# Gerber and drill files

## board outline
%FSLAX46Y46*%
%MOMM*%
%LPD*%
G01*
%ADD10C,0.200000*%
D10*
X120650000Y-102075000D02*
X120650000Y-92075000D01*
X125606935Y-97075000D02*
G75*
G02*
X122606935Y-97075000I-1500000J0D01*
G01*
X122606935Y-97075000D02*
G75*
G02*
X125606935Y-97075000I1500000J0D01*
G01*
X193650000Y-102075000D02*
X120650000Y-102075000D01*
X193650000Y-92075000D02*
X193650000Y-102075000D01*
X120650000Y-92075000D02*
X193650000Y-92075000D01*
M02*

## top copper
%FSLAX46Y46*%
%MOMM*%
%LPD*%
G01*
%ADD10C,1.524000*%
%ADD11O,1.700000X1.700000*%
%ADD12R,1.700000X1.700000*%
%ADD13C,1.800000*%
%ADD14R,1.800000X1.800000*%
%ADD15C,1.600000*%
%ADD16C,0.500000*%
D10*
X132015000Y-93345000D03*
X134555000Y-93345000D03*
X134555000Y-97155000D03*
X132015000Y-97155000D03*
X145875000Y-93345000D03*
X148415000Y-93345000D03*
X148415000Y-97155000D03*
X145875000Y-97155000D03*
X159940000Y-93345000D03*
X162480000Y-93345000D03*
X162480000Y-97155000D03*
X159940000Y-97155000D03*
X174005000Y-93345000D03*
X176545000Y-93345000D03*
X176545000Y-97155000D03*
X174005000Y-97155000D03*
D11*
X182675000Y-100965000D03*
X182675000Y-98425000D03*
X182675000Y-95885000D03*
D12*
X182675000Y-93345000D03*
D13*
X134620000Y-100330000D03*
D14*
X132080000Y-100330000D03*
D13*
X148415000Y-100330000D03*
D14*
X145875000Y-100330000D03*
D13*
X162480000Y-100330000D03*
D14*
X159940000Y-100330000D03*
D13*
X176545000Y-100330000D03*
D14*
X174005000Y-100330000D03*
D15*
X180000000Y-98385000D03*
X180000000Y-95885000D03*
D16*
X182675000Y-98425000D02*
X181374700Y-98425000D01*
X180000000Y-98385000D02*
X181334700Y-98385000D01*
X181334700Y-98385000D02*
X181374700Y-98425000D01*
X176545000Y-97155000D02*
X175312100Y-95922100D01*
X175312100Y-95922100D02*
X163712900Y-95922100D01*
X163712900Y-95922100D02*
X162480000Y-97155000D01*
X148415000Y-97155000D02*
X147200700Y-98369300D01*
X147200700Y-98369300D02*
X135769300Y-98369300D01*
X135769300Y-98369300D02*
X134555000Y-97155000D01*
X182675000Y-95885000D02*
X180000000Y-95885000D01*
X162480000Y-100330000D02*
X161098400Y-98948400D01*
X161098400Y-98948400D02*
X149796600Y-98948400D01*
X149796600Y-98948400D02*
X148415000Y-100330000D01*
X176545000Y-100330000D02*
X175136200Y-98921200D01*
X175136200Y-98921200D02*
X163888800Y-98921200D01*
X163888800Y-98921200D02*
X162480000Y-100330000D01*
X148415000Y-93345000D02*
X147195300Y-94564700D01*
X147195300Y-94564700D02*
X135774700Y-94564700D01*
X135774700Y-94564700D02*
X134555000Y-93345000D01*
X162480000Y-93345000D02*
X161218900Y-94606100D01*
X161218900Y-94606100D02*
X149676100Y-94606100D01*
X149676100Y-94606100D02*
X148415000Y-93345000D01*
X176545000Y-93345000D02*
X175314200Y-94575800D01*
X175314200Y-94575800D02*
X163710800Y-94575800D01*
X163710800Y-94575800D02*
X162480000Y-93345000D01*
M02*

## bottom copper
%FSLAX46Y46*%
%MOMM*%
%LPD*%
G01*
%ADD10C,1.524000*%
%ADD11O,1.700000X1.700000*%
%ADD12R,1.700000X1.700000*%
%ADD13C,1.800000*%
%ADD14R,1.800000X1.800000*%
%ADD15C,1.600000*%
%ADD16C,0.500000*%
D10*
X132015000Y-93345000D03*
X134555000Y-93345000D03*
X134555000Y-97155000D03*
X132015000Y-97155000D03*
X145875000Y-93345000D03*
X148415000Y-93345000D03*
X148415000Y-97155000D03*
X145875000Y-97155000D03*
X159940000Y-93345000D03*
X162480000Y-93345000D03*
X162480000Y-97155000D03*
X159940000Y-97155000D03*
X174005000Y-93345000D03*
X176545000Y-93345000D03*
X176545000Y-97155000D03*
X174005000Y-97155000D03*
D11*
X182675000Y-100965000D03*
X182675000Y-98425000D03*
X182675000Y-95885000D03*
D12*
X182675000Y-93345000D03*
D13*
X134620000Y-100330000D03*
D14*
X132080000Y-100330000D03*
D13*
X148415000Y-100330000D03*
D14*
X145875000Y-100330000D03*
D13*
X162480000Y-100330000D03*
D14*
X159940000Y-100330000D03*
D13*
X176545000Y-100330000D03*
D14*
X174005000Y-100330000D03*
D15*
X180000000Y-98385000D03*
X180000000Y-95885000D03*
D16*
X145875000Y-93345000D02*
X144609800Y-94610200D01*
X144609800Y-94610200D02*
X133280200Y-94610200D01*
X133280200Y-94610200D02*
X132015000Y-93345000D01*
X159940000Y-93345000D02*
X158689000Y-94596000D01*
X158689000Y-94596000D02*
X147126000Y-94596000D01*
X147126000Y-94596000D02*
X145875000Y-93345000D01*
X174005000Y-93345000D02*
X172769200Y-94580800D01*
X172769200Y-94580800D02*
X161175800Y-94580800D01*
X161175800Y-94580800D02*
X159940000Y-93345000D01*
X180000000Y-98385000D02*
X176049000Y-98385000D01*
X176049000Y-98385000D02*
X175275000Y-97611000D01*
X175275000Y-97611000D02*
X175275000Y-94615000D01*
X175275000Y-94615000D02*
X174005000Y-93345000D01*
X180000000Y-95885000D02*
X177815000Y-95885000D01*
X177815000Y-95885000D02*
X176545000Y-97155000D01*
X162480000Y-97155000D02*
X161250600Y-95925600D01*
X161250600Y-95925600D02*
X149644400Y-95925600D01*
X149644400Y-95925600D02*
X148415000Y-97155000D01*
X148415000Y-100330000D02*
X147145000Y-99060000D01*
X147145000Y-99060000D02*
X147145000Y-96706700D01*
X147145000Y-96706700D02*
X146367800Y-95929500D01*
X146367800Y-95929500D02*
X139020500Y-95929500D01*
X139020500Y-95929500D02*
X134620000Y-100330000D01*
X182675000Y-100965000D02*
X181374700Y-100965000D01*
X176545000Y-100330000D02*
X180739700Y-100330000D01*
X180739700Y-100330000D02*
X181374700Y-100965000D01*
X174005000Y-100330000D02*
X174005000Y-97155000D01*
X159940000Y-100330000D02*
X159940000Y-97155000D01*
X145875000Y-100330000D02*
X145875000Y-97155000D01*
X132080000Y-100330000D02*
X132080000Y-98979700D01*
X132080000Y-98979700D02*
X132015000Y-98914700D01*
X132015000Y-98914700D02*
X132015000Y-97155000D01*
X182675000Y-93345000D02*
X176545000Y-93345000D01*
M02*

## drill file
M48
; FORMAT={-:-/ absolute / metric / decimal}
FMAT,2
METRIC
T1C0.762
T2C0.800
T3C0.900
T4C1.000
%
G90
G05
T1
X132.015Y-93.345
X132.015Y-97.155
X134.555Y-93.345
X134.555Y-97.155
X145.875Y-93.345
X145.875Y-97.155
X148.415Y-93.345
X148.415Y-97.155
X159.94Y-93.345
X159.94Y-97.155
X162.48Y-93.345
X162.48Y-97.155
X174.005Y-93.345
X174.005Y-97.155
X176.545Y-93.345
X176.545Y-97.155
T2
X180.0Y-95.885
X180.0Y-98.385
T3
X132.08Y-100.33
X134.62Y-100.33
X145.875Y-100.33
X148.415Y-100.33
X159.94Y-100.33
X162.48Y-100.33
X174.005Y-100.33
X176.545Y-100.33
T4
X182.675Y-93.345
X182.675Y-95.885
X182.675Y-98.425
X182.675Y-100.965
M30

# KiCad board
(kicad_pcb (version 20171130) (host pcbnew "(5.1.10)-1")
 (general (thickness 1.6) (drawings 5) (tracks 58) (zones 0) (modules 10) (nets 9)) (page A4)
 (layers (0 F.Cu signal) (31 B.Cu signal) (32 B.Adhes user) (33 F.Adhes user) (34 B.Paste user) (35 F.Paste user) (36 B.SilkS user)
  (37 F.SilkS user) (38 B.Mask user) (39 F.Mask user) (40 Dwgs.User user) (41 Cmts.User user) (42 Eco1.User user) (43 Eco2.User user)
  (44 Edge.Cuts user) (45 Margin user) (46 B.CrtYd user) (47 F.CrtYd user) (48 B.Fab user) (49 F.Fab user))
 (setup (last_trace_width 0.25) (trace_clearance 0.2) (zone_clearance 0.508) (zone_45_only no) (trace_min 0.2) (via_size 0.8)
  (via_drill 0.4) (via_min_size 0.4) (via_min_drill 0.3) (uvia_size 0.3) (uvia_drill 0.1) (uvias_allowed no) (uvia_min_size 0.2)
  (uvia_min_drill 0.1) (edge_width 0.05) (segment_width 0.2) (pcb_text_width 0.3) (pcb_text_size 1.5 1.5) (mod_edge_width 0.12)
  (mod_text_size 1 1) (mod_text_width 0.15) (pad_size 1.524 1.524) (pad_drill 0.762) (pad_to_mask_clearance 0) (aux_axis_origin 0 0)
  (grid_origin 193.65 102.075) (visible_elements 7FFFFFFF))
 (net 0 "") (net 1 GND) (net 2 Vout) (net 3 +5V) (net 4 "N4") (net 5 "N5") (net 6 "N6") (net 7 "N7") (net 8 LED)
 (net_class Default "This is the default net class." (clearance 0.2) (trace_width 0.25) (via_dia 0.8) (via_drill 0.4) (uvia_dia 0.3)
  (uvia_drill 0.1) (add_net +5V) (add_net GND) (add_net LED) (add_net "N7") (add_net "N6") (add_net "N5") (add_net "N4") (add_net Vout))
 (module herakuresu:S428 (layer F.Cu) (at 133.285 94.615 180)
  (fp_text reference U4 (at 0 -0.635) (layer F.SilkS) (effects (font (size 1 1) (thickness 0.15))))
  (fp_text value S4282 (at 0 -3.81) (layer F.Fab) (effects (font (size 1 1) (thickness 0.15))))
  (pad 4 thru_hole circle (at 1.27 1.27 180) (size 1.524 1.524) (drill 0.762) (layers *.Cu *.Mask) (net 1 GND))
  (pad 3 thru_hole circle (at -1.27 1.27 180) (size 1.524 1.524) (drill 0.762) (layers *.Cu *.Mask) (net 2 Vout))
  (pad 2 thru_hole circle (at -1.27 -2.54 180) (size 1.524 1.524) (drill 0.762) (layers *.Cu *.Mask) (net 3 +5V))
  (pad 1 thru_hole circle (at 1.27 -2.54 180) (size 1.524 1.524) (drill 0.762) (layers *.Cu *.Mask) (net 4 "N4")))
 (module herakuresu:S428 (layer F.Cu) (at 147.145 94.615 180)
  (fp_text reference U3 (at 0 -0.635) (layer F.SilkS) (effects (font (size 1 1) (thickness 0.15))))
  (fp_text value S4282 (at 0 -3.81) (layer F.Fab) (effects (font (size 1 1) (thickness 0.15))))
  (pad 4 thru_hole circle (at 1.27 1.27 180) (size 1.524 1.524) (drill 0.762) (layers *.Cu *.Mask) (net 1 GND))
  (pad 3 thru_hole circle (at -1.27 1.27 180) (size 1.524 1.524) (drill 0.762) (layers *.Cu *.Mask) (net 2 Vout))
  (pad 2 thru_hole circle (at -1.27 -2.54 180) (size 1.524 1.524) (drill 0.762) (layers *.Cu *.Mask) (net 3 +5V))
  (pad 1 thru_hole circle (at 1.27 -2.54 180) (size 1.524 1.524) (drill 0.762) (layers *.Cu *.Mask) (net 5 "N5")))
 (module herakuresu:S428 (layer F.Cu) (at 161.21 94.615 180)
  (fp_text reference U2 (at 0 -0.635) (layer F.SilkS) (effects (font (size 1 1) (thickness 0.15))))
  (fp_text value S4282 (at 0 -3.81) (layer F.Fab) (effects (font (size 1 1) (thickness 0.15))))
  (pad 4 thru_hole circle (at 1.27 1.27 180) (size 1.524 1.524) (drill 0.762) (layers *.Cu *.Mask) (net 1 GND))
  (pad 3 thru_hole circle (at -1.27 1.27 180) (size 1.524 1.524) (drill 0.762) (layers *.Cu *.Mask) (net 2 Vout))
  (pad 2 thru_hole circle (at -1.27 -2.54 180) (size 1.524 1.524) (drill 0.762) (layers *.Cu *.Mask) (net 3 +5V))
  (pad 1 thru_hole circle (at 1.27 -2.54 180) (size 1.524 1.524) (drill 0.762) (layers *.Cu *.Mask) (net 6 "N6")))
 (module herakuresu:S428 (layer F.Cu) (at 175.275 94.615 180)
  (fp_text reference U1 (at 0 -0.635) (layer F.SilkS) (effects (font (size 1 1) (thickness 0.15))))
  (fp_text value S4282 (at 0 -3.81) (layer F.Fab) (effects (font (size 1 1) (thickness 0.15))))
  (pad 4 thru_hole circle (at 1.27 1.27 180) (size 1.524 1.524) (drill 0.762) (layers *.Cu *.Mask) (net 1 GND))
  (pad 3 thru_hole circle (at -1.27 1.27 180) (size 1.524 1.524) (drill 0.762) (layers *.Cu *.Mask) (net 2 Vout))
  (pad 2 thru_hole circle (at -1.27 -2.54 180) (size 1.524 1.524) (drill 0.762) (layers *.Cu *.Mask) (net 3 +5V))
  (pad 1 thru_hole circle (at 1.27 -2.54 180) (size 1.524 1.524) (drill 0.762) (layers *.Cu *.Mask) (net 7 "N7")))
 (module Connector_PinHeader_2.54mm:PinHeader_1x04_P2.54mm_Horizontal (layer F.Cu) (at 182.675 93.345)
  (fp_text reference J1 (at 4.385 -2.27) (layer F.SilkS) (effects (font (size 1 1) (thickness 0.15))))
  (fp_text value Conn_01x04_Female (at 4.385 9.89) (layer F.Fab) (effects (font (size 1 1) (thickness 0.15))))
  (pad 4 thru_hole oval (at 0 7.62) (size 1.7 1.7) (drill 1) (layers *.Cu *.Mask) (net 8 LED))
  (pad 3 thru_hole oval (at 0 5.08) (size 1.7 1.7) (drill 1) (layers *.Cu *.Mask) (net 1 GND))
  (pad 2 thru_hole oval (at 0 2.54) (size 1.7 1.7) (drill 1) (layers *.Cu *.Mask) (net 3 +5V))
  (pad 1 thru_hole rect (at 0 0) (size 1.7 1.7) (drill 1) (layers *.Cu *.Mask) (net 2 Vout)))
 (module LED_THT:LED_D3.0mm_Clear (layer F.Cu) (at 132.08 100.33)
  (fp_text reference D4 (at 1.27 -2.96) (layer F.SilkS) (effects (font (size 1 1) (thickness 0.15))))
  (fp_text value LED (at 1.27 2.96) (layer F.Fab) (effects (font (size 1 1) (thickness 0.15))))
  (pad 2 thru_hole circle (at 2.54 0) (size 1.8 1.8) (drill 0.9) (layers *.Cu *.Mask) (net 8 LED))
  (pad 1 thru_hole rect (at 0 0) (size 1.8 1.8) (drill 0.9) (layers *.Cu *.Mask) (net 4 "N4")))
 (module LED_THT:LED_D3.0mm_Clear (layer F.Cu) (at 145.875 100.33)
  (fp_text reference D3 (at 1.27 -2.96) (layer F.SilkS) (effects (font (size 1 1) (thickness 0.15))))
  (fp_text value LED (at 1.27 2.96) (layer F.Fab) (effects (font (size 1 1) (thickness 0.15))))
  (pad 2 thru_hole circle (at 2.54 0) (size 1.8 1.8) (drill 0.9) (layers *.Cu *.Mask) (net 8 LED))
  (pad 1 thru_hole rect (at 0 0) (size 1.8 1.8) (drill 0.9) (layers *.Cu *.Mask) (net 5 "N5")))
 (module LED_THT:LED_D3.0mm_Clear (layer F.Cu) (at 159.94 100.33)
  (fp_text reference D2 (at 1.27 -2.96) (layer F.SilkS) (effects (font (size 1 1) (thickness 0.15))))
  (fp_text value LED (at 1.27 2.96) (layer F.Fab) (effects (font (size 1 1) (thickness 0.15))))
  (pad 2 thru_hole circle (at 2.54 0) (size 1.8 1.8) (drill 0.9) (layers *.Cu *.Mask) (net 8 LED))
  (pad 1 thru_hole rect (at 0 0) (size 1.8 1.8) (drill 0.9) (layers *.Cu *.Mask) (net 6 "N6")))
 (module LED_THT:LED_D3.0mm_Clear (layer F.Cu) (at 174.005 100.33)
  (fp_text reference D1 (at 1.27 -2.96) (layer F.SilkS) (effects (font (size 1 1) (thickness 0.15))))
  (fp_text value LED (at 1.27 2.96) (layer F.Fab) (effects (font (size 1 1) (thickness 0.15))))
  (pad 2 thru_hole circle (at 2.54 0) (size 1.8 1.8) (drill 0.9) (layers *.Cu *.Mask) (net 8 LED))
  (pad 1 thru_hole rect (at 0 0) (size 1.8 1.8) (drill 0.9) (layers *.Cu *.Mask) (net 7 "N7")))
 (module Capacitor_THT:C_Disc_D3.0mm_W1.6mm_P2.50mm (layer F.Cu) (at 180 95.885 270)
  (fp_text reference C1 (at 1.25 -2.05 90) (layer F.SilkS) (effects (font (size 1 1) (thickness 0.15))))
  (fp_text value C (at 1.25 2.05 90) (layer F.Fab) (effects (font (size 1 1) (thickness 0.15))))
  (pad 2 thru_hole circle (at 2.5 0 270) (size 1.6 1.6) (drill 0.8) (layers *.Cu *.Mask) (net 1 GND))
  (pad 1 thru_hole circle (at 0 0 270) (size 1.6 1.6) (drill 0.8) (layers *.Cu *.Mask) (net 3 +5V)))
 (gr_line (start 120.65 102.075) (end 120.65 92.075) (layer Edge.Cuts) (width 0.2))
 (gr_circle (center 124.106935 97.075) (end 125.606935 97.075) (layer Edge.Cuts) (width 0.2))
 (gr_line (start 193.65 102.075) (end 120.65 102.075) (layer Edge.Cuts) (width 0.2))
 (gr_line (start 193.65 92.075) (end 193.65 102.075) (layer Edge.Cuts) (width 0.2))
 (gr_line (start 120.65 92.075) (end 193.65 92.075) (layer Edge.Cuts) (width 0.2))
 (segment (start 145.875 93.345) (end 144.6098 94.6102) (width 0.5) (layer B.Cu) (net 1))
 (segment (start 144.6098 94.6102) (end 133.2802 94.6102) (width 0.5) (layer B.Cu) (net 1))
 (segment (start 133.2802 94.6102) (end 132.015 93.345) (width 0.5) (layer B.Cu) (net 1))
 (segment (start 159.94 93.345) (end 158.689 94.596) (width 0.5) (layer B.Cu) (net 1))
 (segment (start 158.689 94.596) (end 147.126 94.596) (width 0.5) (layer B.Cu) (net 1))
 (segment (start 147.126 94.596) (end 145.875 93.345) (width 0.5) (layer B.Cu) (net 1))
 (segment (start 174.005 93.345) (end 172.7692 94.5808) (width 0.5) (layer B.Cu) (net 1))
 (segment (start 172.7692 94.5808) (end 161.1758 94.5808) (width 0.5) (layer B.Cu) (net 1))
 (segment (start 161.1758 94.5808) (end 159.94 93.345) (width 0.5) (layer B.Cu) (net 1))
 (segment (start 180 98.385) (end 176.049 98.385) (width 0.5) (layer B.Cu) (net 1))
 (segment (start 176.049 98.385) (end 175.275 97.611) (width 0.5) (layer B.Cu) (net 1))
 (segment (start 175.275 97.611) (end 175.275 94.615) (width 0.5) (layer B.Cu) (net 1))
 (segment (start 175.275 94.615) (end 174.005 93.345) (width 0.5) (layer B.Cu) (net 1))
 (segment (start 182.675 98.425) (end 181.3747 98.425) (width 0.5) (layer F.Cu) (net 1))
 (segment (start 180 98.385) (end 181.3347 98.385) (width 0.5) (layer F.Cu) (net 1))
 (segment (start 181.3347 98.385) (end 181.3747 98.425) (width 0.5) (layer F.Cu) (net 1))
 (segment (start 180 95.885) (end 177.815 95.885) (width 0.5) (layer B.Cu) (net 3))
 (segment (start 177.815 95.885) (end 176.545 97.155) (width 0.5) (layer B.Cu) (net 3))
 (segment (start 176.545 97.155) (end 175.3121 95.9221) (width 0.5) (layer F.Cu) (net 3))
 (segment (start 175.3121 95.9221) (end 163.7129 95.9221) (width 0.5) (layer F.Cu) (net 3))
 (segment (start 163.7129 95.9221) (end 162.48 97.155) (width 0.5) (layer F.Cu) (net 3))
 (segment (start 162.48 97.155) (end 161.2506 95.9256) (width 0.5) (layer B.Cu) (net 3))
 (segment (start 161.2506 95.9256) (end 149.6444 95.9256) (width 0.5) (layer B.Cu) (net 3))
 (segment (start 149.6444 95.9256) (end 148.415 97.155) (width 0.5) (layer B.Cu) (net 3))
 (segment (start 148.415 97.155) (end 147.2007 98.3693) (width 0.5) (layer F.Cu) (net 3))
 (segment (start 147.2007 98.3693) (end 135.7693 98.3693) (width 0.5) (layer F.Cu) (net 3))
 (segment (start 135.7693 98.3693) (end 134.555 97.155) (width 0.5) (layer F.Cu) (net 3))
 (segment (start 182.675 95.885) (end 180 95.885) (width 0.5) (layer F.Cu) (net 3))
 (segment (start 148.415 100.33) (end 147.145 99.06) (width 0.5) (layer B.Cu) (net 8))
 (segment (start 147.145 99.06) (end 147.145 96.7067) (width 0.5) (layer B.Cu) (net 8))
 (segment (start 147.145 96.7067) (end 146.3678 95.9295) (width 0.5) (layer B.Cu) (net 8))
 (segment (start 146.3678 95.9295) (end 139.0205 95.9295) (width 0.5) (layer B.Cu) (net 8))
 (segment (start 139.0205 95.9295) (end 134.62 100.33) (width 0.5) (layer B.Cu) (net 8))
 (segment (start 162.48 100.33) (end 161.0984 98.9484) (width 0.5) (layer F.Cu) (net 8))
 (segment (start 161.0984 98.9484) (end 149.7966 98.9484) (width 0.5) (layer F.Cu) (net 8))
 (segment (start 149.7966 98.9484) (end 148.415 100.33) (width 0.5) (layer F.Cu) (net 8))
 (segment (start 176.545 100.33) (end 175.1362 98.9212) (width 0.5) (layer F.Cu) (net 8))
 (segment (start 175.1362 98.9212) (end 163.8888 98.9212) (width 0.5) (layer F.Cu) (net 8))
 (segment (start 163.8888 98.9212) (end 162.48 100.33) (width 0.5) (layer F.Cu) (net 8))
 (segment (start 182.675 100.965) (end 181.3747 100.965) (width 0.5) (layer B.Cu) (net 8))
 (segment (start 176.545 100.33) (end 180.7397 100.33) (width 0.5) (layer B.Cu) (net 8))
 (segment (start 180.7397 100.33) (end 181.3747 100.965) (width 0.5) (layer B.Cu) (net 8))
 (segment (start 174.005 100.33) (end 174.005 97.155) (width 0.5) (layer B.Cu) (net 7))
 (segment (start 159.94 100.33) (end 159.94 97.155) (width 0.5) (layer B.Cu) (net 6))
 (segment (start 145.875 100.33) (end 145.875 97.155) (width 0.5) (layer B.Cu) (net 5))
 (segment (start 132.08 100.33) (end 132.08 98.9797) (width 0.5) (layer B.Cu) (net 4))
 (segment (start 132.08 98.9797) (end 132.015 98.9147) (width 0.5) (layer B.Cu) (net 4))
 (segment (start 132.015 98.9147) (end 132.015 97.155) (width 0.5) (layer B.Cu) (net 4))
 (segment (start 148.415 93.345) (end 147.1953 94.5647) (width 0.5) (layer F.Cu) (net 2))
 (segment (start 147.1953 94.5647) (end 135.7747 94.5647) (width 0.5) (layer F.Cu) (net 2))
 (segment (start 135.7747 94.5647) (end 134.555 93.345) (width 0.5) (layer F.Cu) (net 2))
 (segment (start 162.48 93.345) (end 161.2189 94.6061) (width 0.5) (layer F.Cu) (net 2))
 (segment (start 161.2189 94.6061) (end 149.6761 94.6061) (width 0.5) (layer F.Cu) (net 2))
 (segment (start 149.6761 94.6061) (end 148.415 93.345) (width 0.5) (layer F.Cu) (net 2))
 (segment (start 176.545 93.345) (end 175.3142 94.5758) (width 0.5) (layer F.Cu) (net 2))
 (segment (start 175.3142 94.5758) (end 163.7108 94.5758) (width 0.5) (layer F.Cu) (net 2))
 (segment (start 163.7108 94.5758) (end 162.48 93.345) (width 0.5) (layer F.Cu) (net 2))
 (segment (start 182.675 93.345) (end 176.545 93.345) (width 0.5) (layer B.Cu) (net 2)))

